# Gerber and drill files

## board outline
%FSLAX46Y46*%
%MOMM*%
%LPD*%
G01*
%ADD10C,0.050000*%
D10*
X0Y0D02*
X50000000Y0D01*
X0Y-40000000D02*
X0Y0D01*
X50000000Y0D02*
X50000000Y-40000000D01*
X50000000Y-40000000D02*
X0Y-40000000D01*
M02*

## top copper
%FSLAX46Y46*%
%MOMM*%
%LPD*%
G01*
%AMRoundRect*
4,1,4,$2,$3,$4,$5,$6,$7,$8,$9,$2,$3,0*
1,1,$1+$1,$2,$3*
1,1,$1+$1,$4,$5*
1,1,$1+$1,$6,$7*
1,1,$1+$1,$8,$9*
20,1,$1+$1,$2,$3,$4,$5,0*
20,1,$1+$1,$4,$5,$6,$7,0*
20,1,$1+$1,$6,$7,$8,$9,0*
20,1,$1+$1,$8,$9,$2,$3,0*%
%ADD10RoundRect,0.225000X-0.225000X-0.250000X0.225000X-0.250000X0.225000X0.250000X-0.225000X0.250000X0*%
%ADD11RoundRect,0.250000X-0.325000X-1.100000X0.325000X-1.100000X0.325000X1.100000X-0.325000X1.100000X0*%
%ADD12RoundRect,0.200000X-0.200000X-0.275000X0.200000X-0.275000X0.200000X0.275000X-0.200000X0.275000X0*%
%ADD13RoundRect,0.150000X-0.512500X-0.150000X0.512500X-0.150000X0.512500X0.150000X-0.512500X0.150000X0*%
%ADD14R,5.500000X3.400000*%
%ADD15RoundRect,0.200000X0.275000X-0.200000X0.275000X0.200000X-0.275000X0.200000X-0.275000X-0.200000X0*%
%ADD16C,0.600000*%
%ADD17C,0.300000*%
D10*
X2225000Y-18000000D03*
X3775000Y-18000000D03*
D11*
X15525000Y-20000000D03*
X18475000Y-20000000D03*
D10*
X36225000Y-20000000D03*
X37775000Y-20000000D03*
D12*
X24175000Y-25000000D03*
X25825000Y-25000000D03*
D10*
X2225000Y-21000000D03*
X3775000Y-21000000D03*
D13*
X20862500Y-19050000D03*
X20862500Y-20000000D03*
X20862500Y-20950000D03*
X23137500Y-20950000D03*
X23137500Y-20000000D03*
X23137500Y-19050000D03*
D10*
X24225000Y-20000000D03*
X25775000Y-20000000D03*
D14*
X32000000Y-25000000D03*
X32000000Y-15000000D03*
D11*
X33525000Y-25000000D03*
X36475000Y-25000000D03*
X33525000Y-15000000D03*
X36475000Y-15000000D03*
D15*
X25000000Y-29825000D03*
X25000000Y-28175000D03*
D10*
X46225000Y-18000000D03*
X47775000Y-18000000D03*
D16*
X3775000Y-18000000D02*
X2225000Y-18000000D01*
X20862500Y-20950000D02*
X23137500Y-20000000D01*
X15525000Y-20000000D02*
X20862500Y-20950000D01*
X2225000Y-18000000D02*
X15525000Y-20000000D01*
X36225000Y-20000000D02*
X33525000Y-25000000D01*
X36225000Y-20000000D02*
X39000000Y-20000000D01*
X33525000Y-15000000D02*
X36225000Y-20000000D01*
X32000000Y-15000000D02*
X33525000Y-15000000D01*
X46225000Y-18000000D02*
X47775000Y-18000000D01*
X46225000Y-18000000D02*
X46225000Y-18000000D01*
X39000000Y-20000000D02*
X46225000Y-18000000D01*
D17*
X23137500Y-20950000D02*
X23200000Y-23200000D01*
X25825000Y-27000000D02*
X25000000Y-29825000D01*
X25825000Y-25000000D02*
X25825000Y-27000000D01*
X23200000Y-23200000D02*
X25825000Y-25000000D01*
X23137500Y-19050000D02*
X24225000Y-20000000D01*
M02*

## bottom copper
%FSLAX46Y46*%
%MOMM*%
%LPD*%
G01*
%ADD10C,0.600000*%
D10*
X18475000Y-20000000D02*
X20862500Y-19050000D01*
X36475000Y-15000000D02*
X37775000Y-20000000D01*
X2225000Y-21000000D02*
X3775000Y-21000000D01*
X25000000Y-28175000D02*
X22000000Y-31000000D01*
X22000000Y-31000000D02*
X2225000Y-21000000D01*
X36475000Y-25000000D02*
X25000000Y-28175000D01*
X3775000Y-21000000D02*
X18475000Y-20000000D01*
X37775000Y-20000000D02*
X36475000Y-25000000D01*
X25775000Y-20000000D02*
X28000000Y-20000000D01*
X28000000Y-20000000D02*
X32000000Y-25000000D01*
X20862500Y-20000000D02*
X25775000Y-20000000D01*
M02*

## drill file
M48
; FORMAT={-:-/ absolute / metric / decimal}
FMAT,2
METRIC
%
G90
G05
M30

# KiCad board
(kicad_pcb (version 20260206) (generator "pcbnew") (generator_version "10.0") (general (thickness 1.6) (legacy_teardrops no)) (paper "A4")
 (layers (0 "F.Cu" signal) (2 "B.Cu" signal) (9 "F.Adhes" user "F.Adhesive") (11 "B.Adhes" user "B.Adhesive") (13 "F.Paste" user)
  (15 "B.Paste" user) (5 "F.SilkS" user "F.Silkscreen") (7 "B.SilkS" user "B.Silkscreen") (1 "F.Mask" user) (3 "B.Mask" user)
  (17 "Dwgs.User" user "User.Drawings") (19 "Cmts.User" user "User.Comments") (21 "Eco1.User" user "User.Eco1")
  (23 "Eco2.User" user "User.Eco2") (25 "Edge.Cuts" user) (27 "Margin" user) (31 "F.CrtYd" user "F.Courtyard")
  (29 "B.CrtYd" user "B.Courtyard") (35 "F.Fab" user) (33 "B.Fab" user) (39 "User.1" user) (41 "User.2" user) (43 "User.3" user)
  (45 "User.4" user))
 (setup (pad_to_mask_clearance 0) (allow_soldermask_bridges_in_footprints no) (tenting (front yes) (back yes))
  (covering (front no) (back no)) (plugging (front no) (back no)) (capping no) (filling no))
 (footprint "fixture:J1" (layer "F.Cu") (at 3 18)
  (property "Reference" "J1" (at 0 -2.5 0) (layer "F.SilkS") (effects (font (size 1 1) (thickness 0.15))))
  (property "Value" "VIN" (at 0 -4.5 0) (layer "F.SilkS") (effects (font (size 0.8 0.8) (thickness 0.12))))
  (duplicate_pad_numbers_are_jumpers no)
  (pad "1" smd roundrect (at -0.775 0) (size 0.9 0.95) (layers "F.Cu" "F.Mask" "F.Paste") (roundrect_rratio 0.25) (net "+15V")
   (thermal_bridge_angle 45))
  (pad "2" smd roundrect (at 0.775 0) (size 0.9 0.95) (layers "F.Cu" "F.Mask" "F.Paste") (roundrect_rratio 0.25) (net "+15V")
   (thermal_bridge_angle 45)))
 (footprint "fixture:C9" (layer "F.Cu") (at 17 20)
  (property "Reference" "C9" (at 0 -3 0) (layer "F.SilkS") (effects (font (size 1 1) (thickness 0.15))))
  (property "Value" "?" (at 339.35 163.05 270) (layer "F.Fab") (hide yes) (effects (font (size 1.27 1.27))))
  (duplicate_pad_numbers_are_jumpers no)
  (pad "1" smd roundrect (at -1.475 0) (size 1.15 2.7) (layers "F.Cu" "F.Mask" "F.Paste") (roundrect_rratio 0.217391) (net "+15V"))
  (pad "2" smd roundrect (at 1.475 0) (size 1.15 2.7) (layers "F.Cu" "F.Mask" "F.Paste") (roundrect_rratio 0.217391) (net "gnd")))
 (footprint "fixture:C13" (layer "F.Cu") (at 37 20)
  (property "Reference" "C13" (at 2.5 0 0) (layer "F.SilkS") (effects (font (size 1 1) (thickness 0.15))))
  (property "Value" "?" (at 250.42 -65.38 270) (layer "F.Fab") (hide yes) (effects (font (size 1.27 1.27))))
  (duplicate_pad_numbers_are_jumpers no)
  (pad "1" smd roundrect (at -0.775 0) (size 0.9 0.95) (layers "F.Cu" "F.Mask" "F.Paste") (roundrect_rratio 0.25) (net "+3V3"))
  (pad "2" smd roundrect (at 0.775 0) (size 0.9 0.95) (layers "F.Cu" "F.Mask" "F.Paste") (roundrect_rratio 0.25) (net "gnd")))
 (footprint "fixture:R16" (layer "F.Cu") (at 25 25)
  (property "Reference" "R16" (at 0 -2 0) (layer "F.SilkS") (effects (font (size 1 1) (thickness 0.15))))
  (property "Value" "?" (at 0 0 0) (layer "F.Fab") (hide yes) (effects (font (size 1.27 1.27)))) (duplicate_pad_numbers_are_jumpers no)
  (pad "1" smd roundrect (at -0.825 0) (size 0.8 0.95) (layers "F.Cu" "F.Mask" "F.Paste") (roundrect_rratio 0.25) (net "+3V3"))
  (pad "2" smd roundrect (at 0.825 0) (size 0.8 0.95) (layers "F.Cu" "F.Mask" "F.Paste") (roundrect_rratio 0.25) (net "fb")))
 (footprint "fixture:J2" (layer "F.Cu") (at 3 21)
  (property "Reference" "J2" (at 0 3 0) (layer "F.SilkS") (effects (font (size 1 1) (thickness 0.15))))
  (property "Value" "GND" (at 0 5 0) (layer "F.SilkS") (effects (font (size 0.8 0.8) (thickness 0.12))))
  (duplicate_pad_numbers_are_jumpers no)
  (pad "1" smd roundrect (at -0.775 0) (size 0.9 0.95) (layers "F.Cu" "F.Mask" "F.Paste") (roundrect_rratio 0.25) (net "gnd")
   (thermal_bridge_angle 45))
  (pad "2" smd roundrect (at 0.775 0) (size 0.9 0.95) (layers "F.Cu" "F.Mask" "F.Paste") (roundrect_rratio 0.25) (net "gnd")
   (thermal_bridge_angle 45)))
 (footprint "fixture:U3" (layer "F.Cu") (at 22 20)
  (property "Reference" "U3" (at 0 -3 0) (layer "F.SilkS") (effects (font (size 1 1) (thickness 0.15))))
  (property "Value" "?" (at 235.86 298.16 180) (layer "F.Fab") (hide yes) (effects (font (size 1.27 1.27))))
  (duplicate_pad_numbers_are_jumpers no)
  (pad "1" smd roundrect (at -1.1375 -0.95) (size 1.325 0.6) (layers "F.Cu" "F.Mask" "F.Paste") (roundrect_rratio 0.25) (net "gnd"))
  (pad "2" smd roundrect (at -1.1375 0) (size 1.325 0.6) (layers "F.Cu" "F.Mask" "F.Paste") (roundrect_rratio 0.25) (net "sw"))
  (pad "3" smd roundrect (at -1.1375 0.95) (size 1.325 0.6) (layers "F.Cu" "F.Mask" "F.Paste") (roundrect_rratio 0.25) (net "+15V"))
  (pad "4" smd roundrect (at 1.1375 0.95) (size 1.325 0.6) (layers "F.Cu" "F.Mask" "F.Paste") (roundrect_rratio 0.25) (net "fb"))
  (pad "5" smd roundrect (at 1.1375 0) (size 1.325 0.6) (layers "F.Cu" "F.Mask" "F.Paste") (roundrect_rratio 0.25) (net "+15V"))
  (pad "6" smd roundrect (at 1.1375 -0.95) (size 1.325 0.6) (layers "F.Cu" "F.Mask" "F.Paste") (roundrect_rratio 0.25) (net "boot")))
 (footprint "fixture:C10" (layer "F.Cu") (at 25 20)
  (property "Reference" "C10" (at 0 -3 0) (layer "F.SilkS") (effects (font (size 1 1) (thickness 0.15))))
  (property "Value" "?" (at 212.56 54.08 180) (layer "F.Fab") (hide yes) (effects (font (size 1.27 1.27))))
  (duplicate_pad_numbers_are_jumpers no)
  (pad "1" smd roundrect (at -0.775 0) (size 0.9 0.95) (layers "F.Cu" "F.Mask" "F.Paste") (roundrect_rratio 0.25) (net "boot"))
  (pad "2" smd roundrect (at 0.775 0) (size 0.9 0.95) (layers "F.Cu" "F.Mask" "F.Paste") (roundrect_rratio 0.25) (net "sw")))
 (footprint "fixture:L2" (layer "F.Cu") (at 32 20 90)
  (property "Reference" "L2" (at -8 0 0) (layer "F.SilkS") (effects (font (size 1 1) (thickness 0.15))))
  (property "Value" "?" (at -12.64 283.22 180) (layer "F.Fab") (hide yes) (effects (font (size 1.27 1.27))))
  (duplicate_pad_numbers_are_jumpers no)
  (pad "1" smd rect (at -5 0 90) (size 3.4 5.5) (layers "F.Cu" "F.Mask" "F.Paste") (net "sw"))
  (pad "2" smd rect (at 5 0 90) (size 3.4 5.5) (layers "F.Cu" "F.Mask" "F.Paste") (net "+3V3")))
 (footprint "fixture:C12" (layer "F.Cu") (at 35 25)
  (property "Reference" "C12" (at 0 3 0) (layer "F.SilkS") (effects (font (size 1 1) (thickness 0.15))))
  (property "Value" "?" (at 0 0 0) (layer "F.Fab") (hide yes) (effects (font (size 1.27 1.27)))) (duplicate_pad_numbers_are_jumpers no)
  (pad "1" smd roundrect (at -1.475 0) (size 1.15 2.7) (layers "F.Cu" "F.Mask" "F.Paste") (roundrect_rratio 0.217391) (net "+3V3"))
  (pad "2" smd roundrect (at 1.475 0) (size 1.15 2.7) (layers "F.Cu" "F.Mask" "F.Paste") (roundrect_rratio 0.217391) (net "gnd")))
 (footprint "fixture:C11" (layer "F.Cu") (at 35 15)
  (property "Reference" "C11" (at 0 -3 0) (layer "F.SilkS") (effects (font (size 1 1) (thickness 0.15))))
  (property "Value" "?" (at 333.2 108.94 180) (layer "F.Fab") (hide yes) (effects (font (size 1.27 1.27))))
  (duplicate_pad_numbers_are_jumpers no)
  (pad "1" smd roundrect (at -1.475 0) (size 1.15 2.7) (layers "F.Cu" "F.Mask" "F.Paste") (roundrect_rratio 0.217391) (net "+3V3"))
  (pad "2" smd roundrect (at 1.475 0) (size 1.15 2.7) (layers "F.Cu" "F.Mask" "F.Paste") (roundrect_rratio 0.217391) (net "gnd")))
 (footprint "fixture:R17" (layer "F.Cu") (at 25 29 90)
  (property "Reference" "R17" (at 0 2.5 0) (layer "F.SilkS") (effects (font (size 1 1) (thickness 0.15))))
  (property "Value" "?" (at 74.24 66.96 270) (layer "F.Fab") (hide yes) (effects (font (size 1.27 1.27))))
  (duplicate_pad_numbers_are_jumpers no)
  (pad "1" smd roundrect (at -0.825 0 90) (size 0.8 0.95) (layers "F.Cu" "F.Mask" "F.Paste") (roundrect_rratio 0.25) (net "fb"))
  (pad "2" smd roundrect (at 0.825 0 90) (size 0.8 0.95) (layers "F.Cu" "F.Mask" "F.Paste") (roundrect_rratio 0.25) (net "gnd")))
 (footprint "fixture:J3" (layer "F.Cu") (at 47 18)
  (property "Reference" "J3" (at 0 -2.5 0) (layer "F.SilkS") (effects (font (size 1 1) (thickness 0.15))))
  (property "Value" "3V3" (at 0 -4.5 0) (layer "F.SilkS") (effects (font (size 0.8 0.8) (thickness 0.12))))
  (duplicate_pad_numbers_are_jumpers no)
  (pad "1" smd roundrect (at -0.775 0) (size 0.9 0.95) (layers "F.Cu" "F.Mask" "F.Paste") (roundrect_rratio 0.25) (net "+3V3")
   (thermal_bridge_angle 45))
  (pad "2" smd roundrect (at 0.775 0) (size 0.9 0.95) (layers "F.Cu" "F.Mask" "F.Paste") (roundrect_rratio 0.25) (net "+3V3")
   (thermal_bridge_angle 45)))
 (gr_line (start 0 0) (end 50 0) (stroke (width 0.05) (type default)) (layer "Edge.Cuts"))
 (gr_line (start 0 40) (end 0 0) (stroke (width 0.05) (type default)) (layer "Edge.Cuts"))
 (gr_line (start 50 0) (end 50 40) (stroke (width 0.05) (type default)) (layer "Edge.Cuts"))
 (gr_line (start 50 40) (end 0 40) (stroke (width 0.05) (type default)) (layer "Edge.Cuts"))
 (segment (start 3.775 18) (end 2.225 18) (width 0.6) (layer "F.Cu") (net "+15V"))
 (segment (start 20.8625 20.95) (end 23.1375 20) (width 0.6) (layer "F.Cu") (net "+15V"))
 (segment (start 15.525 20) (end 20.8625 20.95) (width 0.6) (layer "F.Cu") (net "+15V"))
 (segment (start 2.225 18) (end 15.525 20) (width 0.6) (layer "F.Cu") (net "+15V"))
 (segment (start 18.475 20) (end 20.8625 19.05) (width 0.6) (layer "B.Cu") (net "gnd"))
 (segment (start 36.475 15) (end 37.775 20) (width 0.6) (layer "B.Cu") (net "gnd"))
 (segment (start 2.225 21) (end 3.775 21) (width 0.6) (layer "B.Cu") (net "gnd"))
 (segment (start 25 28.175) (end 22 31) (width 0.6) (layer "B.Cu") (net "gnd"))
 (segment (start 22 31) (end 2.225 21) (width 0.6) (layer "B.Cu") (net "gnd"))
 (segment (start 36.475 25) (end 25 28.175) (width 0.6) (layer "B.Cu") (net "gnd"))
 (segment (start 3.775 21) (end 18.475 20) (width 0.6) (layer "B.Cu") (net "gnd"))
 (segment (start 37.775 20) (end 36.475 25) (width 0.6) (layer "B.Cu") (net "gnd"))
 (segment (start 36.225 20) (end 33.525 25) (width 0.6) (layer "F.Cu") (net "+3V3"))
 (segment (start 36.225 20) (end 39 20) (width 0.6) (layer "F.Cu") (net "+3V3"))
 (segment (start 33.525 15) (end 36.225 20) (width 0.6) (layer "F.Cu") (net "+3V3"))
 (segment (start 32 15) (end 33.525 15) (width 0.6) (layer "F.Cu") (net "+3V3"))
 (segment (start 46.225 18) (end 47.775 18) (width 0.6) (layer "F.Cu") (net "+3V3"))
 (segment (start 46.225 18) (end 46.225 18) (width 0.6) (layer "F.Cu") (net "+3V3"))
 (segment (start 39 20) (end 46.225 18) (width 0.6) (layer "F.Cu") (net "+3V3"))
 (segment (start 23.1375 20.95) (end 23.2 23.2) (width 0.3) (layer "F.Cu") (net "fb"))
 (segment (start 25.825 27) (end 25 29.825) (width 0.3) (layer "F.Cu") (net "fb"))
 (segment (start 25.825 25) (end 25.825 27) (width 0.3) (layer "F.Cu") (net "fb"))
 (segment (start 23.2 23.2) (end 25.825 25) (width 0.3) (layer "F.Cu") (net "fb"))
 (segment (start 25.775 20) (end 28 20) (width 0.6) (layer "B.Cu") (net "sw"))
 (segment (start 28 20) (end 32 25) (width 0.6) (layer "B.Cu") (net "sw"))
 (segment (start 20.8625 20) (end 25.775 20) (width 0.6) (layer "B.Cu") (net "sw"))
 (segment (start 23.1375 19.05) (end 24.225 20) (width 0.3) (layer "F.Cu") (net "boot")))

